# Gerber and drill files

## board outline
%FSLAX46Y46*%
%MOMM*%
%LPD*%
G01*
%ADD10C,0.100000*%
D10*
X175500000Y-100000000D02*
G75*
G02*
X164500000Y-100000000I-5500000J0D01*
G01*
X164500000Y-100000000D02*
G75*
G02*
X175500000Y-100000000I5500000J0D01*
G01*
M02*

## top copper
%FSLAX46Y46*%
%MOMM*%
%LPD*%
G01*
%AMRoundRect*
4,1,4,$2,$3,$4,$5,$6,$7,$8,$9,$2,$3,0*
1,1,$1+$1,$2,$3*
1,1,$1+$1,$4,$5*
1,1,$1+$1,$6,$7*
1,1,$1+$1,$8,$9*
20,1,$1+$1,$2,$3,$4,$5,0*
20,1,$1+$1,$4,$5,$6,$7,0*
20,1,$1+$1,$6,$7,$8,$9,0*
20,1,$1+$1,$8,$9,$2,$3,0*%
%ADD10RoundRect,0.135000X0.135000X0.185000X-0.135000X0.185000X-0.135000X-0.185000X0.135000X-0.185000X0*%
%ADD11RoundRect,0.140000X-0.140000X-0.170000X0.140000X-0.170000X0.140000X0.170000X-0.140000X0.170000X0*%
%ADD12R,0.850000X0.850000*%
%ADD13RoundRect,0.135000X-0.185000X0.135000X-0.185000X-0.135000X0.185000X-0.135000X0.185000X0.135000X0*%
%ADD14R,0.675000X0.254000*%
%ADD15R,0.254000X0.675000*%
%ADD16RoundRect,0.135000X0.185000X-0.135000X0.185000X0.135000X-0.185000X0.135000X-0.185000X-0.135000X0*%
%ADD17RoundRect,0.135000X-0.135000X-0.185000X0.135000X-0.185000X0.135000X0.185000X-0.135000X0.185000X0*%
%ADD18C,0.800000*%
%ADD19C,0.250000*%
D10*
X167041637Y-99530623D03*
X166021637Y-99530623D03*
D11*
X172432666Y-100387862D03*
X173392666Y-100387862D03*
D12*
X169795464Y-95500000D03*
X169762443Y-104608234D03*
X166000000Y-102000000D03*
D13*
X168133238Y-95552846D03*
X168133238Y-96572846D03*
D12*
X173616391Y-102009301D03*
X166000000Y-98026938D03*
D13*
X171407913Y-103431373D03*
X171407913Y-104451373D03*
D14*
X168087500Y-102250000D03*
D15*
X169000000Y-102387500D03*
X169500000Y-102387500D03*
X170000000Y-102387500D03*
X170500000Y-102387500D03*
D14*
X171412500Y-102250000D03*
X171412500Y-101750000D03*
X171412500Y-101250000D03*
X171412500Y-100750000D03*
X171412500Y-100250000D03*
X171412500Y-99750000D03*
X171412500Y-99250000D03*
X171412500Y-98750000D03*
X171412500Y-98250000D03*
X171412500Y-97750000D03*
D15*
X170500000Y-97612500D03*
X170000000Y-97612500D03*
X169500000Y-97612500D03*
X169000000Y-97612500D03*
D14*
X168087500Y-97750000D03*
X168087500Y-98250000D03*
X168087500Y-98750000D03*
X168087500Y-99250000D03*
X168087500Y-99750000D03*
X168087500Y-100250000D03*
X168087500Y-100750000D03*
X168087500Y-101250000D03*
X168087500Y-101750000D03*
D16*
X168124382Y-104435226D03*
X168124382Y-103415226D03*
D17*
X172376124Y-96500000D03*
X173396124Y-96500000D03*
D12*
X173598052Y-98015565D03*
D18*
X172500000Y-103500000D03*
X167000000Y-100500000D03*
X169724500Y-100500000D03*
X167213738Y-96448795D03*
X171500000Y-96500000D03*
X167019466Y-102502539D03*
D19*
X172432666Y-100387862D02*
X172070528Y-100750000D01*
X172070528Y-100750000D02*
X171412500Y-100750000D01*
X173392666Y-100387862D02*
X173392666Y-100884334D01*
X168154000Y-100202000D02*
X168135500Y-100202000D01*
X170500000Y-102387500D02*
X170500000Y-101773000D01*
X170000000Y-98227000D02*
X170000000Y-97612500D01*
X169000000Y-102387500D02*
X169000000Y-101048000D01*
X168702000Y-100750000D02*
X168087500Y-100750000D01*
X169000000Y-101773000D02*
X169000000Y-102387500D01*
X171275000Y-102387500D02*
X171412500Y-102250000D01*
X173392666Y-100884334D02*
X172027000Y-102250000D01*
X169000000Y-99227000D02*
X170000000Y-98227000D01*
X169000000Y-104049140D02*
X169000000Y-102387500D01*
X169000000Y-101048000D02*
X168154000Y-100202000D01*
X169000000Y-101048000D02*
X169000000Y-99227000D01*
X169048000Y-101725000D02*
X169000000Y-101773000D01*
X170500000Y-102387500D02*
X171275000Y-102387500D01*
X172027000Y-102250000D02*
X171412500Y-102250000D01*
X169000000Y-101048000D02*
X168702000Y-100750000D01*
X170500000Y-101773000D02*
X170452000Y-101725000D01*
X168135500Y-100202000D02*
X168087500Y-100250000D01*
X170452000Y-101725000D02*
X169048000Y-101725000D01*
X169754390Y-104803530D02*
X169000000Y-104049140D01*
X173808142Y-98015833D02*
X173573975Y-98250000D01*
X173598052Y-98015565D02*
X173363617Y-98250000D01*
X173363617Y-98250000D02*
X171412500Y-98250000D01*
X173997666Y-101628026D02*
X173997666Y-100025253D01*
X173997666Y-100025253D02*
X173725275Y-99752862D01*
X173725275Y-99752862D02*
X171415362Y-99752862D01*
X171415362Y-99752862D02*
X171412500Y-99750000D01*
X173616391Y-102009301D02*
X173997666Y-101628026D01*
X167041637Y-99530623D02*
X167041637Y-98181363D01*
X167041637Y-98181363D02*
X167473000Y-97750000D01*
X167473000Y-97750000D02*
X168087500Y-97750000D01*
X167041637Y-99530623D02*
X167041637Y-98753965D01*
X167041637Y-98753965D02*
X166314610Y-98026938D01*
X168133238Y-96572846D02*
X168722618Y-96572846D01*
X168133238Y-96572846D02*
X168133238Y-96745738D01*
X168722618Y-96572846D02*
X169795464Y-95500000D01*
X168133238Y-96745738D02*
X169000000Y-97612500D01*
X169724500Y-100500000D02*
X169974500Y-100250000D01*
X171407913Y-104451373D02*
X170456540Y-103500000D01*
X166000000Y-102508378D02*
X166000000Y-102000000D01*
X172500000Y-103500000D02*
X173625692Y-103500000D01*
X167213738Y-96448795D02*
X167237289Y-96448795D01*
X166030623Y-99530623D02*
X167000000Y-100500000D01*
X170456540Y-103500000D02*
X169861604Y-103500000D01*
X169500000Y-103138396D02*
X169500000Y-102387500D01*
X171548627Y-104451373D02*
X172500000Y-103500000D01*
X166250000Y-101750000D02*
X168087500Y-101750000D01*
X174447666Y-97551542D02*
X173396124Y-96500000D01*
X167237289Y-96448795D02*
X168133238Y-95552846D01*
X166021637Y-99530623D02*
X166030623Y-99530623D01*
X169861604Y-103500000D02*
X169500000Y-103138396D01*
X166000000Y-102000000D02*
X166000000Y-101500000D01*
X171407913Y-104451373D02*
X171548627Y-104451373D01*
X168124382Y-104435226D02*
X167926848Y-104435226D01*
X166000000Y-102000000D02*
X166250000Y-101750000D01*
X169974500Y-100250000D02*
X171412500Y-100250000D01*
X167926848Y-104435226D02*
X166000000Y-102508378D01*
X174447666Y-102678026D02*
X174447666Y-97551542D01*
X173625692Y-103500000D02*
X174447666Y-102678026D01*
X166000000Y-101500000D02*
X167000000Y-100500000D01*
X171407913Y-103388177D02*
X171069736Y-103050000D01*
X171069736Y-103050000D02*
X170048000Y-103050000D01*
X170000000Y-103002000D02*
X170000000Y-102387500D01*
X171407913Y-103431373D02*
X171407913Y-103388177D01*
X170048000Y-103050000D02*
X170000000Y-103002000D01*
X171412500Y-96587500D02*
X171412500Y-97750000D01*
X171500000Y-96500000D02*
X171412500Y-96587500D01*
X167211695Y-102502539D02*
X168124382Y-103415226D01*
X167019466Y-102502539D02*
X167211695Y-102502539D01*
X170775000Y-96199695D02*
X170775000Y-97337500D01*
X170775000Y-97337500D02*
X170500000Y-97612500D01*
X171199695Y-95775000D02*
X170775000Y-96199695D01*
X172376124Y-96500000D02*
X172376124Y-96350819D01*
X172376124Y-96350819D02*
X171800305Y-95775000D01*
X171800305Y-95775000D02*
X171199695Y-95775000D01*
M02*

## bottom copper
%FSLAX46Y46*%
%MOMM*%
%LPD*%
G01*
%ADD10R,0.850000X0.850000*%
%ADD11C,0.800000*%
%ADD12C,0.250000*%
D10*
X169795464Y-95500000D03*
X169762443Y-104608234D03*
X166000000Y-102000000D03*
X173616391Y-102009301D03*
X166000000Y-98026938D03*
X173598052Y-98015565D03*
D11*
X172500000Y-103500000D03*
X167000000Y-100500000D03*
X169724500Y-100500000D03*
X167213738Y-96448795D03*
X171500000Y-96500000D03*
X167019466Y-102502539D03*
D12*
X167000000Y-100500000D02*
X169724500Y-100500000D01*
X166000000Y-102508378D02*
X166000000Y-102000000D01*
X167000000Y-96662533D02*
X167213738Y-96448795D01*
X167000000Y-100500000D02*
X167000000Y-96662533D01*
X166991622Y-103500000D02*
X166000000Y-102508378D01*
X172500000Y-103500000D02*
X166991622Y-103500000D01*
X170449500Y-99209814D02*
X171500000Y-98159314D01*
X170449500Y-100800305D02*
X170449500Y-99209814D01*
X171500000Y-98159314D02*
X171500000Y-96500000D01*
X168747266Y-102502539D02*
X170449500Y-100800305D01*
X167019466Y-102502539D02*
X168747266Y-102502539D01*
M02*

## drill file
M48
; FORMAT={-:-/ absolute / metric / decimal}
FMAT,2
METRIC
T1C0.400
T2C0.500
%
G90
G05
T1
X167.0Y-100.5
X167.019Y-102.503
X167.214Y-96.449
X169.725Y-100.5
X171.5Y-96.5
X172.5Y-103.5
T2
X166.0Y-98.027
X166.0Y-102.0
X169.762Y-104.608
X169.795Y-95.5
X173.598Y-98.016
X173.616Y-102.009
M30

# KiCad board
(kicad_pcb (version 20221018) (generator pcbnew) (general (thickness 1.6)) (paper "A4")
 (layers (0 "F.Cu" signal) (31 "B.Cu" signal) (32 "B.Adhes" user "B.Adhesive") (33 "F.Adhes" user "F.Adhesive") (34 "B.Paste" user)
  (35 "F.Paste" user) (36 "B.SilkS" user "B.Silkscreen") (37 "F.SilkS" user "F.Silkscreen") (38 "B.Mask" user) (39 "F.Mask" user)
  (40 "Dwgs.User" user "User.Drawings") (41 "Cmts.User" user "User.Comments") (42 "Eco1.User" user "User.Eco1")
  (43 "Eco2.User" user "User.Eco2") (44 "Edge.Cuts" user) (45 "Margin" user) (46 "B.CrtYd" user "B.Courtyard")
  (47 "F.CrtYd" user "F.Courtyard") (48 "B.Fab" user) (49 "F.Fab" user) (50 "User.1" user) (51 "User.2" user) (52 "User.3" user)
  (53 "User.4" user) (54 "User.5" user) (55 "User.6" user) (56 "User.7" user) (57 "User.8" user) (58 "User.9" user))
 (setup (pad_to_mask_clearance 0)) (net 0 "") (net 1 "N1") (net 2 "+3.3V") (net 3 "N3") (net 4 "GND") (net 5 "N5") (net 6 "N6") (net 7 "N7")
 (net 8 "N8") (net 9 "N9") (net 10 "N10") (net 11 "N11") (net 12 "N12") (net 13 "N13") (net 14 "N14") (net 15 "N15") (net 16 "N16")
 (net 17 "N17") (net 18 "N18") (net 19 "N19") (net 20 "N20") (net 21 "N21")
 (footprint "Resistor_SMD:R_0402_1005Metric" (layer "F.Cu") (at 166.531637 99.530623 180)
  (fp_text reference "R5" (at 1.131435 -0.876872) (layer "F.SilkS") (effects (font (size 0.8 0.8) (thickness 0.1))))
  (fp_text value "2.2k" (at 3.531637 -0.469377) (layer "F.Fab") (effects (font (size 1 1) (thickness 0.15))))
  (pad "1" smd roundrect (at -0.51 0 180) (size 0.54 0.64) (layers "F.Cu" "F.Paste" "F.Mask") (roundrect_rratio 0.25) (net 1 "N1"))
  (pad "2" smd roundrect (at 0.51 0 180) (size 0.54 0.64) (layers "F.Cu" "F.Paste" "F.Mask") (roundrect_rratio 0.25) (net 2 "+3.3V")))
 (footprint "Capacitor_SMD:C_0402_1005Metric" (layer "F.Cu") (at 172.912666 100.387862)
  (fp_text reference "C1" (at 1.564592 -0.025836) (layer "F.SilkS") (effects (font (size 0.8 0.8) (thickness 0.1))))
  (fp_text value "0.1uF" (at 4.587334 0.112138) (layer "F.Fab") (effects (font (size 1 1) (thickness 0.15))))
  (pad "1" smd roundrect (at -0.48 0) (size 0.56 0.62) (layers "F.Cu" "F.Paste" "F.Mask") (roundrect_rratio 0.25) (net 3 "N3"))
  (pad "2" smd roundrect (at 0.48 0) (size 0.56 0.62) (layers "F.Cu" "F.Paste" "F.Mask") (roundrect_rratio 0.25) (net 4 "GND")))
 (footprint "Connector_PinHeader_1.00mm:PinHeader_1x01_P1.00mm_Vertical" (layer "F.Cu") (at 169.795464 95.5)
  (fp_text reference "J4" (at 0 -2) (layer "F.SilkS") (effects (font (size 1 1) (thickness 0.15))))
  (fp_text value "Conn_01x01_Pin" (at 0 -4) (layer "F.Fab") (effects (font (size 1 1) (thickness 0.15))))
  (pad "1" thru_hole rect (at 0 0) (size 0.85 0.85) (drill 0.5) (layers "*.Cu" "*.Mask") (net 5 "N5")))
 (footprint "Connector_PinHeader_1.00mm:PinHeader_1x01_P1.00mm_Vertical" (layer "F.Cu") (at 169.762443 104.608234)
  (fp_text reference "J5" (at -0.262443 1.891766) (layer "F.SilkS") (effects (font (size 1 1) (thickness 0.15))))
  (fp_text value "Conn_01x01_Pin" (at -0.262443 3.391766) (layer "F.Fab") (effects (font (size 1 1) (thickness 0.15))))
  (pad "1" thru_hole rect (at 0 0) (size 0.85 0.85) (drill 0.5) (layers "*.Cu" "*.Mask") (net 4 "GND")))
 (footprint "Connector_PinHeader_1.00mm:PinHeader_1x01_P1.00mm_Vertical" (layer "F.Cu") (at 166 102)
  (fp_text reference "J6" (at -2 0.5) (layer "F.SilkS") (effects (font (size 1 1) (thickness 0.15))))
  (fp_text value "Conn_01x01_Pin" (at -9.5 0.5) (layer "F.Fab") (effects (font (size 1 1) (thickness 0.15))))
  (pad "1" thru_hole rect (at 0 0) (size 0.85 0.85) (drill 0.5) (layers "*.Cu" "*.Mask") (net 2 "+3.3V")))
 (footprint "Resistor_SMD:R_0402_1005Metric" (layer "F.Cu") (at 168.133238 96.062846 -90)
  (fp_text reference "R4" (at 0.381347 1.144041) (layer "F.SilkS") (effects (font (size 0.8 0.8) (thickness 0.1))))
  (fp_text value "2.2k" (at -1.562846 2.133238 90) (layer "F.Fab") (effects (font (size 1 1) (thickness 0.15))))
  (pad "1" smd roundrect (at -0.51 0 270) (size 0.54 0.64) (layers "F.Cu" "F.Paste" "F.Mask") (roundrect_rratio 0.25) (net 2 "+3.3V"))
  (pad "2" smd roundrect (at 0.51 0 270) (size 0.54 0.64) (layers "F.Cu" "F.Paste" "F.Mask") (roundrect_rratio 0.25) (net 5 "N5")))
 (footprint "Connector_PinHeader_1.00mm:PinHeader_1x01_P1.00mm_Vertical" (layer "F.Cu") (at 173.616391 102.009301)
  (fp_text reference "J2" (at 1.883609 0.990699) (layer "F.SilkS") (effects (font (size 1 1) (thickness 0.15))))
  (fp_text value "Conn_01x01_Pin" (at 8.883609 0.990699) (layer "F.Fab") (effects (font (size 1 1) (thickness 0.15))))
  (pad "1" thru_hole rect (at 0 0) (size 0.85 0.85) (drill 0.5) (layers "*.Cu" "*.Mask") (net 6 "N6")))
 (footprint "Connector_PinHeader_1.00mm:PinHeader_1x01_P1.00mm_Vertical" (layer "F.Cu") (at 166 98.026938)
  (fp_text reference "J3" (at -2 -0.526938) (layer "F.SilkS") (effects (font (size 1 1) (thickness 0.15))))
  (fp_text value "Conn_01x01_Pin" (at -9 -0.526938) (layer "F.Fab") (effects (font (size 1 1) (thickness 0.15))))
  (pad "1" thru_hole rect (at 0 0) (size 0.85 0.85) (drill 0.5) (layers "*.Cu" "*.Mask") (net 1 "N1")))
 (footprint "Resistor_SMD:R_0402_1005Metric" (layer "F.Cu") (at 171.407913 103.941373 -90)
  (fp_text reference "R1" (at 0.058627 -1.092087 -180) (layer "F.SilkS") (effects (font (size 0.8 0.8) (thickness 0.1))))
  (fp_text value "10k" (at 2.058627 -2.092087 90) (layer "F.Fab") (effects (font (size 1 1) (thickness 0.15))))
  (pad "1" smd roundrect (at -0.51 0 270) (size 0.54 0.64) (layers "F.Cu" "F.Paste" "F.Mask") (roundrect_rratio 0.25) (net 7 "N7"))
  (pad "2" smd roundrect (at 0.51 0 270) (size 0.54 0.64) (layers "F.Cu" "F.Paste" "F.Mask") (roundrect_rratio 0.25) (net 2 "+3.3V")))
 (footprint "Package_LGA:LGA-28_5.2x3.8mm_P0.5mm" (layer "F.Cu") (at 169.75 100 90)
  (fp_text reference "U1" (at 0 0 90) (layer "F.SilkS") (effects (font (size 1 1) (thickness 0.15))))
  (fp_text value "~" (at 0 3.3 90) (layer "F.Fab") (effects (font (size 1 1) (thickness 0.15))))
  (pad "1" smd rect (at -2.25 -1.6625 90) (size 0.254 0.675) (layers "F.Cu" "F.Paste" "F.Mask") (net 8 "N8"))
  (pad "2" smd rect (at -2.3875 -0.75 180) (size 0.254 0.675) (layers "F.Cu" "F.Paste" "F.Mask") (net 4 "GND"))
  (pad "3" smd rect (at -2.3875 -0.25 180) (size 0.254 0.675) (layers "F.Cu" "F.Paste" "F.Mask") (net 2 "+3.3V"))
  (pad "4" smd rect (at -2.3875 0.25 180) (size 0.254 0.675) (layers "F.Cu" "F.Paste" "F.Mask") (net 7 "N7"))
  (pad "5" smd rect (at -2.3875 0.75 180) (size 0.254 0.675) (layers "F.Cu" "F.Paste" "F.Mask") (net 4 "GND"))
  (pad "6" smd rect (at -2.25 1.6625 90) (size 0.254 0.675) (layers "F.Cu" "F.Paste" "F.Mask") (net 4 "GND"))
  (pad "7" smd rect (at -1.75 1.6625 90) (size 0.254 0.675) (layers "F.Cu" "F.Paste" "F.Mask") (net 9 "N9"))
  (pad "8" smd rect (at -1.25 1.6625 90) (size 0.254 0.675) (layers "F.Cu" "F.Paste" "F.Mask") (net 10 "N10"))
  (pad "9" smd rect (at -0.75 1.6625 90) (size 0.254 0.675) (layers "F.Cu" "F.Paste" "F.Mask") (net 3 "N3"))
  (pad "10" smd rect (at -0.25 1.6625 90) (size 0.254 0.675) (layers "F.Cu" "F.Paste" "F.Mask") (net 2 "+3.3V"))
  (pad "11" smd rect (at 0.25 1.6625 90) (size 0.254 0.675) (layers "F.Cu" "F.Paste" "F.Mask") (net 6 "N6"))
  (pad "12" smd rect (at 0.75 1.6625 90) (size 0.254 0.675) (layers "F.Cu" "F.Paste" "F.Mask") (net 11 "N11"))
  (pad "13" smd rect (at 1.25 1.6625 90) (size 0.254 0.675) (layers "F.Cu" "F.Paste" "F.Mask") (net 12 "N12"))
  (pad "14" smd rect (at 1.75 1.6625 90) (size 0.254 0.675) (layers "F.Cu" "F.Paste" "F.Mask") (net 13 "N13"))
  (pad "15" smd rect (at 2.25 1.6625 90) (size 0.254 0.675) (layers "F.Cu" "F.Paste" "F.Mask") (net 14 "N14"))
  (pad "16" smd rect (at 2.3875 0.75 180) (size 0.254 0.675) (layers "F.Cu" "F.Paste" "F.Mask") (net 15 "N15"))
  (pad "17" smd rect (at 2.3875 0.25 180) (size 0.254 0.675) (layers "F.Cu" "F.Paste" "F.Mask") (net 4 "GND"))
  (pad "18" smd rect (at 2.3875 -0.25 180) (size 0.254 0.675) (layers "F.Cu" "F.Paste" "F.Mask") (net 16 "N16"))
  (pad "19" smd rect (at 2.3875 -0.75 180) (size 0.254 0.675) (layers "F.Cu" "F.Paste" "F.Mask") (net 5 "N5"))
  (pad "20" smd rect (at 2.25 -1.6625 90) (size 0.254 0.675) (layers "F.Cu" "F.Paste" "F.Mask") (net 1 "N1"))
  (pad "21" smd rect (at 1.75 -1.6625 90) (size 0.254 0.675) (layers "F.Cu" "F.Paste" "F.Mask") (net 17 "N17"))
  (pad "22" smd rect (at 1.25 -1.6625 90) (size 0.254 0.675) (layers "F.Cu" "F.Paste" "F.Mask") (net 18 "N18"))
  (pad "23" smd rect (at 0.75 -1.6625 90) (size 0.254 0.675) (layers "F.Cu" "F.Paste" "F.Mask") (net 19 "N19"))
  (pad "24" smd rect (at 0.25 -1.6625 90) (size 0.254 0.675) (layers "F.Cu" "F.Paste" "F.Mask") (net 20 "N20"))
  (pad "25" smd rect (at -0.25 -1.6625 90) (size 0.254 0.675) (layers "F.Cu" "F.Paste" "F.Mask") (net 4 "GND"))
  (pad "26" smd rect (at -0.75 -1.6625 90) (size 0.254 0.675) (layers "F.Cu" "F.Paste" "F.Mask") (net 4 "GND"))
  (pad "27" smd rect (at -1.25 -1.6625 90) (size 0.254 0.675) (layers "F.Cu" "F.Paste" "F.Mask") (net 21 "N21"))
  (pad "28" smd rect (at -1.75 -1.6625 90) (size 0.254 0.675) (layers "F.Cu" "F.Paste" "F.Mask") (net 2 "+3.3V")))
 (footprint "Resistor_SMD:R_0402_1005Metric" (layer "F.Cu") (at 168.124382 103.925226 90)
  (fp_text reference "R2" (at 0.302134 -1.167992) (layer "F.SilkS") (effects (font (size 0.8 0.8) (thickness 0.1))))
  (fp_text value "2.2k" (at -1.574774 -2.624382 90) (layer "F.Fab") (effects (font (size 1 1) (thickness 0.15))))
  (pad "1" smd roundrect (at -0.51 0 90) (size 0.54 0.64) (layers "F.Cu" "F.Paste" "F.Mask") (roundrect_rratio 0.25) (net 2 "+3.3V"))
  (pad "2" smd roundrect (at 0.51 0 90) (size 0.54 0.64) (layers "F.Cu" "F.Paste" "F.Mask") (roundrect_rratio 0.25) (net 14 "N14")))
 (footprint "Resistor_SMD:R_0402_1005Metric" (layer "F.Cu") (at 172.886124 96.5)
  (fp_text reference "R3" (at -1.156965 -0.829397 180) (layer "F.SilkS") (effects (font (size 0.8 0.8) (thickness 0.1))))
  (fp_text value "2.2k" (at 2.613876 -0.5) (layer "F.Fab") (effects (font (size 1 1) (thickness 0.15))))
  (pad "1" smd roundrect (at -0.51 0) (size 0.54 0.64) (layers "F.Cu" "F.Paste" "F.Mask") (roundrect_rratio 0.25) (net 15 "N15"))
  (pad "2" smd roundrect (at 0.51 0) (size 0.54 0.64) (layers "F.Cu" "F.Paste" "F.Mask") (roundrect_rratio 0.25) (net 2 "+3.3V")))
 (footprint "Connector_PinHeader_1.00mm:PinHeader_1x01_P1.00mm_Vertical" (layer "F.Cu") (at 173.598052 98.015565)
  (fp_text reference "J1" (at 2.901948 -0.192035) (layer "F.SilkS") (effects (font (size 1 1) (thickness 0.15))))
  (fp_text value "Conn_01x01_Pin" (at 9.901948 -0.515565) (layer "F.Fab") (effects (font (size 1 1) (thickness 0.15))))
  (pad "1" thru_hole rect (at 0 0) (size 0.85 0.85) (drill 0.5) (layers "*.Cu" "*.Mask") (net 13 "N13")))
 (gr_circle (center 170 100) (end 175.5 100) (stroke (width 0.1) (type default)) (fill none) (layer "Edge.Cuts"))
 (segment (start 172.432666 100.387862) (end 172.070528 100.75) (width 0.25) (layer "F.Cu") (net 3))
 (segment (start 172.070528 100.75) (end 171.4125 100.75) (width 0.25) (layer "F.Cu") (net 3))
 (segment (start 173.392666 100.387862) (end 173.392666 100.884334) (width 0.25) (layer "F.Cu") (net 4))
 (segment (start 168.154 100.202) (end 168.1355 100.202) (width 0.25) (layer "F.Cu") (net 4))
 (segment (start 170.5 102.3875) (end 170.5 101.773) (width 0.25) (layer "F.Cu") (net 4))
 (segment (start 170 98.227) (end 170 97.6125) (width 0.25) (layer "F.Cu") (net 4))
 (segment (start 169 102.3875) (end 169 101.048) (width 0.25) (layer "F.Cu") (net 4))
 (segment (start 168.702 100.75) (end 168.0875 100.75) (width 0.25) (layer "F.Cu") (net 4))
 (segment (start 169 101.773) (end 169 102.3875) (width 0.25) (layer "F.Cu") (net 4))
 (segment (start 171.275 102.3875) (end 171.4125 102.25) (width 0.25) (layer "F.Cu") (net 4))
 (segment (start 173.392666 100.884334) (end 172.027 102.25) (width 0.25) (layer "F.Cu") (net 4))
 (segment (start 169 99.227) (end 170 98.227) (width 0.25) (layer "F.Cu") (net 4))
 (segment (start 169 104.04914) (end 169 102.3875) (width 0.25) (layer "F.Cu") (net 4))
 (segment (start 169 101.048) (end 168.154 100.202) (width 0.25) (layer "F.Cu") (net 4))
 (segment (start 169 101.048) (end 169 99.227) (width 0.25) (layer "F.Cu") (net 4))
 (segment (start 169.048 101.725) (end 169 101.773) (width 0.25) (layer "F.Cu") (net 4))
 (segment (start 170.5 102.3875) (end 171.275 102.3875) (width 0.25) (layer "F.Cu") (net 4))
 (segment (start 172.027 102.25) (end 171.4125 102.25) (width 0.25) (layer "F.Cu") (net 4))
 (segment (start 169 101.048) (end 168.702 100.75) (width 0.25) (layer "F.Cu") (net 4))
 (segment (start 170.5 101.773) (end 170.452 101.725) (width 0.25) (layer "F.Cu") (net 4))
 (segment (start 168.1355 100.202) (end 168.0875 100.25) (width 0.25) (layer "F.Cu") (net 4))
 (segment (start 170.452 101.725) (end 169.048 101.725) (width 0.25) (layer "F.Cu") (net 4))
 (segment (start 169.75439 104.80353) (end 169 104.04914) (width 0.25) (layer "F.Cu") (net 4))
 (segment (start 173.808142 98.015833) (end 173.573975 98.25) (width 0.25) (layer "F.Cu") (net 13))
 (segment (start 173.598052 98.015565) (end 173.363617 98.25) (width 0.25) (layer "F.Cu") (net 13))
 (segment (start 173.363617 98.25) (end 171.4125 98.25) (width 0.25) (layer "F.Cu") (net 13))
 (segment (start 173.997666 101.628026) (end 173.997666 100.025253) (width 0.25) (layer "F.Cu") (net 6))
 (segment (start 173.997666 100.025253) (end 173.725275 99.752862) (width 0.25) (layer "F.Cu") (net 6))
 (segment (start 173.725275 99.752862) (end 171.415362 99.752862) (width 0.25) (layer "F.Cu") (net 6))
 (segment (start 171.415362 99.752862) (end 171.4125 99.75) (width 0.25) (layer "F.Cu") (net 6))
 (segment (start 173.616391 102.009301) (end 173.997666 101.628026) (width 0.25) (layer "F.Cu") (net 6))
 (segment (start 167.041637 99.530623) (end 167.041637 98.181363) (width 0.25) (layer "F.Cu") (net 1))
 (segment (start 167.041637 98.181363) (end 167.473 97.75) (width 0.25) (layer "F.Cu") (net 1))
 (segment (start 167.473 97.75) (end 168.0875 97.75) (width 0.25) (layer "F.Cu") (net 1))
 (segment (start 167.041637 99.530623) (end 167.041637 98.753965) (width 0.25) (layer "F.Cu") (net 1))
 (segment (start 167.041637 98.753965) (end 166.31461 98.026938) (width 0.25) (layer "F.Cu") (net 1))
 (segment (start 168.133238 96.572846) (end 168.722618 96.572846) (width 0.25) (layer "F.Cu") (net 5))
 (segment (start 168.133238 96.572846) (end 168.133238 96.745738) (width 0.25) (layer "F.Cu") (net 5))
 (segment (start 168.722618 96.572846) (end 169.795464 95.5) (width 0.25) (layer "F.Cu") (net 5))
 (segment (start 168.133238 96.745738) (end 169 97.6125) (width 0.25) (layer "F.Cu") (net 5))
 (segment (start 169.7245 100.5) (end 169.9745 100.25) (width 0.25) (layer "F.Cu") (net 2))
 (segment (start 171.407913 104.451373) (end 170.45654 103.5) (width 0.25) (layer "F.Cu") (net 2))
 (segment (start 166 102.508378) (end 166 102) (width 0.25) (layer "F.Cu") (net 2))
 (segment (start 172.5 103.5) (end 173.625692 103.5) (width 0.25) (layer "F.Cu") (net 2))
 (segment (start 167.213738 96.448795) (end 167.237289 96.448795) (width 0.25) (layer "F.Cu") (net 2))
 (segment (start 166.030623 99.530623) (end 167 100.5) (width 0.25) (layer "F.Cu") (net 2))
 (segment (start 170.45654 103.5) (end 169.861604 103.5) (width 0.25) (layer "F.Cu") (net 2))
 (segment (start 169.5 103.138396) (end 169.5 102.3875) (width 0.25) (layer "F.Cu") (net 2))
 (segment (start 171.548627 104.451373) (end 172.5 103.5) (width 0.25) (layer "F.Cu") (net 2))
 (segment (start 166.25 101.75) (end 168.0875 101.75) (width 0.25) (layer "F.Cu") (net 2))
 (segment (start 174.447666 97.551542) (end 173.396124 96.5) (width 0.25) (layer "F.Cu") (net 2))
 (segment (start 167.237289 96.448795) (end 168.133238 95.552846) (width 0.25) (layer "F.Cu") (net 2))
 (segment (start 166.021637 99.530623) (end 166.030623 99.530623) (width 0.25) (layer "F.Cu") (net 2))
 (segment (start 169.861604 103.5) (end 169.5 103.138396) (width 0.25) (layer "F.Cu") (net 2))
 (segment (start 166 102) (end 166 101.5) (width 0.25) (layer "F.Cu") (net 2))
 (segment (start 171.407913 104.451373) (end 171.548627 104.451373) (width 0.25) (layer "F.Cu") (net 2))
 (segment (start 168.124382 104.435226) (end 167.926848 104.435226) (width 0.25) (layer "F.Cu") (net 2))
 (segment (start 166 102) (end 166.25 101.75) (width 0.25) (layer "F.Cu") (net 2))
 (segment (start 169.9745 100.25) (end 171.4125 100.25) (width 0.25) (layer "F.Cu") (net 2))
 (segment (start 167.926848 104.435226) (end 166 102.508378) (width 0.25) (layer "F.Cu") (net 2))
 (segment (start 174.447666 102.678026) (end 174.447666 97.551542) (width 0.25) (layer "F.Cu") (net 2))
 (segment (start 173.625692 103.5) (end 174.447666 102.678026) (width 0.25) (layer "F.Cu") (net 2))
 (segment (start 166 101.5) (end 167 100.5) (width 0.25) (layer "F.Cu") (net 2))
 (via (at 172.5 103.5) (size 0.8) (drill 0.4) (layers "F.Cu" "B.Cu") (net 2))
 (via (at 167 100.5) (size 0.8) (drill 0.4) (layers "F.Cu" "B.Cu") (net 2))
 (via (at 169.7245 100.5) (size 0.8) (drill 0.4) (layers "F.Cu" "B.Cu") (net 2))
 (via (at 167.213738 96.448795) (size 0.8) (drill 0.4) (layers "F.Cu" "B.Cu") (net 2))
 (segment (start 167 100.5) (end 169.7245 100.5) (width 0.25) (layer "B.Cu") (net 2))
 (segment (start 166 102.508378) (end 166 102) (width 0.25) (layer "B.Cu") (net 2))
 (segment (start 167 96.662533) (end 167.213738 96.448795) (width 0.25) (layer "B.Cu") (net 2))
 (segment (start 167 100.5) (end 167 96.662533) (width 0.25) (layer "B.Cu") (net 2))
 (segment (start 166.991622 103.5) (end 166 102.508378) (width 0.25) (layer "B.Cu") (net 2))
 (segment (start 172.5 103.5) (end 166.991622 103.5) (width 0.25) (layer "B.Cu") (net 2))
 (segment (start 171.407913 103.388177) (end 171.069736 103.05) (width 0.25) (layer "F.Cu") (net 7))
 (segment (start 171.069736 103.05) (end 170.048 103.05) (width 0.25) (layer "F.Cu") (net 7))
 (segment (start 170 103.002) (end 170 102.3875) (width 0.25) (layer "F.Cu") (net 7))
 (segment (start 171.407913 103.431373) (end 171.407913 103.388177) (width 0.25) (layer "F.Cu") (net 7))
 (segment (start 170.048 103.05) (end 170 103.002) (width 0.25) (layer "F.Cu") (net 7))
 (segment (start 171.4125 96.5875) (end 171.4125 97.75) (width 0.25) (layer "F.Cu") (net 14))
 (segment (start 171.5 96.5) (end 171.4125 96.5875) (width 0.25) (layer "F.Cu") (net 14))
 (segment (start 167.211695 102.502539) (end 168.124382 103.415226) (width 0.25) (layer "F.Cu") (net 14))
 (segment (start 167.019466 102.502539) (end 167.211695 102.502539) (width 0.25) (layer "F.Cu") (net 14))
 (via (at 171.5 96.5) (size 0.8) (drill 0.4) (layers "F.Cu" "B.Cu") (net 14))
 (via (at 167.019466 102.502539) (size 0.8) (drill 0.4) (layers "F.Cu" "B.Cu") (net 14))
 (segment (start 170.4495 99.209814) (end 171.5 98.159314) (width 0.25) (layer "B.Cu") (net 14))
 (segment (start 170.4495 100.800305) (end 170.4495 99.209814) (width 0.25) (layer "B.Cu") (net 14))
 (segment (start 171.5 98.159314) (end 171.5 96.5) (width 0.25) (layer "B.Cu") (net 14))
 (segment (start 168.747266 102.502539) (end 170.4495 100.800305) (width 0.25) (layer "B.Cu") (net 14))
 (segment (start 167.019466 102.502539) (end 168.747266 102.502539) (width 0.25) (layer "B.Cu") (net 14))
 (segment (start 170.775 96.199695) (end 170.775 97.3375) (width 0.25) (layer "F.Cu") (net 15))
 (segment (start 170.775 97.3375) (end 170.5 97.6125) (width 0.25) (layer "F.Cu") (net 15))
 (segment (start 171.199695 95.775) (end 170.775 96.199695) (width 0.25) (layer "F.Cu") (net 15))
 (segment (start 172.376124 96.5) (end 172.376124 96.350819) (width 0.25) (layer "F.Cu") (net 15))
 (segment (start 172.376124 96.350819) (end 171.800305 95.775) (width 0.25) (layer "F.Cu") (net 15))
 (segment (start 171.800305 95.775) (end 171.199695 95.775) (width 0.25) (layer "F.Cu") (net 15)))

